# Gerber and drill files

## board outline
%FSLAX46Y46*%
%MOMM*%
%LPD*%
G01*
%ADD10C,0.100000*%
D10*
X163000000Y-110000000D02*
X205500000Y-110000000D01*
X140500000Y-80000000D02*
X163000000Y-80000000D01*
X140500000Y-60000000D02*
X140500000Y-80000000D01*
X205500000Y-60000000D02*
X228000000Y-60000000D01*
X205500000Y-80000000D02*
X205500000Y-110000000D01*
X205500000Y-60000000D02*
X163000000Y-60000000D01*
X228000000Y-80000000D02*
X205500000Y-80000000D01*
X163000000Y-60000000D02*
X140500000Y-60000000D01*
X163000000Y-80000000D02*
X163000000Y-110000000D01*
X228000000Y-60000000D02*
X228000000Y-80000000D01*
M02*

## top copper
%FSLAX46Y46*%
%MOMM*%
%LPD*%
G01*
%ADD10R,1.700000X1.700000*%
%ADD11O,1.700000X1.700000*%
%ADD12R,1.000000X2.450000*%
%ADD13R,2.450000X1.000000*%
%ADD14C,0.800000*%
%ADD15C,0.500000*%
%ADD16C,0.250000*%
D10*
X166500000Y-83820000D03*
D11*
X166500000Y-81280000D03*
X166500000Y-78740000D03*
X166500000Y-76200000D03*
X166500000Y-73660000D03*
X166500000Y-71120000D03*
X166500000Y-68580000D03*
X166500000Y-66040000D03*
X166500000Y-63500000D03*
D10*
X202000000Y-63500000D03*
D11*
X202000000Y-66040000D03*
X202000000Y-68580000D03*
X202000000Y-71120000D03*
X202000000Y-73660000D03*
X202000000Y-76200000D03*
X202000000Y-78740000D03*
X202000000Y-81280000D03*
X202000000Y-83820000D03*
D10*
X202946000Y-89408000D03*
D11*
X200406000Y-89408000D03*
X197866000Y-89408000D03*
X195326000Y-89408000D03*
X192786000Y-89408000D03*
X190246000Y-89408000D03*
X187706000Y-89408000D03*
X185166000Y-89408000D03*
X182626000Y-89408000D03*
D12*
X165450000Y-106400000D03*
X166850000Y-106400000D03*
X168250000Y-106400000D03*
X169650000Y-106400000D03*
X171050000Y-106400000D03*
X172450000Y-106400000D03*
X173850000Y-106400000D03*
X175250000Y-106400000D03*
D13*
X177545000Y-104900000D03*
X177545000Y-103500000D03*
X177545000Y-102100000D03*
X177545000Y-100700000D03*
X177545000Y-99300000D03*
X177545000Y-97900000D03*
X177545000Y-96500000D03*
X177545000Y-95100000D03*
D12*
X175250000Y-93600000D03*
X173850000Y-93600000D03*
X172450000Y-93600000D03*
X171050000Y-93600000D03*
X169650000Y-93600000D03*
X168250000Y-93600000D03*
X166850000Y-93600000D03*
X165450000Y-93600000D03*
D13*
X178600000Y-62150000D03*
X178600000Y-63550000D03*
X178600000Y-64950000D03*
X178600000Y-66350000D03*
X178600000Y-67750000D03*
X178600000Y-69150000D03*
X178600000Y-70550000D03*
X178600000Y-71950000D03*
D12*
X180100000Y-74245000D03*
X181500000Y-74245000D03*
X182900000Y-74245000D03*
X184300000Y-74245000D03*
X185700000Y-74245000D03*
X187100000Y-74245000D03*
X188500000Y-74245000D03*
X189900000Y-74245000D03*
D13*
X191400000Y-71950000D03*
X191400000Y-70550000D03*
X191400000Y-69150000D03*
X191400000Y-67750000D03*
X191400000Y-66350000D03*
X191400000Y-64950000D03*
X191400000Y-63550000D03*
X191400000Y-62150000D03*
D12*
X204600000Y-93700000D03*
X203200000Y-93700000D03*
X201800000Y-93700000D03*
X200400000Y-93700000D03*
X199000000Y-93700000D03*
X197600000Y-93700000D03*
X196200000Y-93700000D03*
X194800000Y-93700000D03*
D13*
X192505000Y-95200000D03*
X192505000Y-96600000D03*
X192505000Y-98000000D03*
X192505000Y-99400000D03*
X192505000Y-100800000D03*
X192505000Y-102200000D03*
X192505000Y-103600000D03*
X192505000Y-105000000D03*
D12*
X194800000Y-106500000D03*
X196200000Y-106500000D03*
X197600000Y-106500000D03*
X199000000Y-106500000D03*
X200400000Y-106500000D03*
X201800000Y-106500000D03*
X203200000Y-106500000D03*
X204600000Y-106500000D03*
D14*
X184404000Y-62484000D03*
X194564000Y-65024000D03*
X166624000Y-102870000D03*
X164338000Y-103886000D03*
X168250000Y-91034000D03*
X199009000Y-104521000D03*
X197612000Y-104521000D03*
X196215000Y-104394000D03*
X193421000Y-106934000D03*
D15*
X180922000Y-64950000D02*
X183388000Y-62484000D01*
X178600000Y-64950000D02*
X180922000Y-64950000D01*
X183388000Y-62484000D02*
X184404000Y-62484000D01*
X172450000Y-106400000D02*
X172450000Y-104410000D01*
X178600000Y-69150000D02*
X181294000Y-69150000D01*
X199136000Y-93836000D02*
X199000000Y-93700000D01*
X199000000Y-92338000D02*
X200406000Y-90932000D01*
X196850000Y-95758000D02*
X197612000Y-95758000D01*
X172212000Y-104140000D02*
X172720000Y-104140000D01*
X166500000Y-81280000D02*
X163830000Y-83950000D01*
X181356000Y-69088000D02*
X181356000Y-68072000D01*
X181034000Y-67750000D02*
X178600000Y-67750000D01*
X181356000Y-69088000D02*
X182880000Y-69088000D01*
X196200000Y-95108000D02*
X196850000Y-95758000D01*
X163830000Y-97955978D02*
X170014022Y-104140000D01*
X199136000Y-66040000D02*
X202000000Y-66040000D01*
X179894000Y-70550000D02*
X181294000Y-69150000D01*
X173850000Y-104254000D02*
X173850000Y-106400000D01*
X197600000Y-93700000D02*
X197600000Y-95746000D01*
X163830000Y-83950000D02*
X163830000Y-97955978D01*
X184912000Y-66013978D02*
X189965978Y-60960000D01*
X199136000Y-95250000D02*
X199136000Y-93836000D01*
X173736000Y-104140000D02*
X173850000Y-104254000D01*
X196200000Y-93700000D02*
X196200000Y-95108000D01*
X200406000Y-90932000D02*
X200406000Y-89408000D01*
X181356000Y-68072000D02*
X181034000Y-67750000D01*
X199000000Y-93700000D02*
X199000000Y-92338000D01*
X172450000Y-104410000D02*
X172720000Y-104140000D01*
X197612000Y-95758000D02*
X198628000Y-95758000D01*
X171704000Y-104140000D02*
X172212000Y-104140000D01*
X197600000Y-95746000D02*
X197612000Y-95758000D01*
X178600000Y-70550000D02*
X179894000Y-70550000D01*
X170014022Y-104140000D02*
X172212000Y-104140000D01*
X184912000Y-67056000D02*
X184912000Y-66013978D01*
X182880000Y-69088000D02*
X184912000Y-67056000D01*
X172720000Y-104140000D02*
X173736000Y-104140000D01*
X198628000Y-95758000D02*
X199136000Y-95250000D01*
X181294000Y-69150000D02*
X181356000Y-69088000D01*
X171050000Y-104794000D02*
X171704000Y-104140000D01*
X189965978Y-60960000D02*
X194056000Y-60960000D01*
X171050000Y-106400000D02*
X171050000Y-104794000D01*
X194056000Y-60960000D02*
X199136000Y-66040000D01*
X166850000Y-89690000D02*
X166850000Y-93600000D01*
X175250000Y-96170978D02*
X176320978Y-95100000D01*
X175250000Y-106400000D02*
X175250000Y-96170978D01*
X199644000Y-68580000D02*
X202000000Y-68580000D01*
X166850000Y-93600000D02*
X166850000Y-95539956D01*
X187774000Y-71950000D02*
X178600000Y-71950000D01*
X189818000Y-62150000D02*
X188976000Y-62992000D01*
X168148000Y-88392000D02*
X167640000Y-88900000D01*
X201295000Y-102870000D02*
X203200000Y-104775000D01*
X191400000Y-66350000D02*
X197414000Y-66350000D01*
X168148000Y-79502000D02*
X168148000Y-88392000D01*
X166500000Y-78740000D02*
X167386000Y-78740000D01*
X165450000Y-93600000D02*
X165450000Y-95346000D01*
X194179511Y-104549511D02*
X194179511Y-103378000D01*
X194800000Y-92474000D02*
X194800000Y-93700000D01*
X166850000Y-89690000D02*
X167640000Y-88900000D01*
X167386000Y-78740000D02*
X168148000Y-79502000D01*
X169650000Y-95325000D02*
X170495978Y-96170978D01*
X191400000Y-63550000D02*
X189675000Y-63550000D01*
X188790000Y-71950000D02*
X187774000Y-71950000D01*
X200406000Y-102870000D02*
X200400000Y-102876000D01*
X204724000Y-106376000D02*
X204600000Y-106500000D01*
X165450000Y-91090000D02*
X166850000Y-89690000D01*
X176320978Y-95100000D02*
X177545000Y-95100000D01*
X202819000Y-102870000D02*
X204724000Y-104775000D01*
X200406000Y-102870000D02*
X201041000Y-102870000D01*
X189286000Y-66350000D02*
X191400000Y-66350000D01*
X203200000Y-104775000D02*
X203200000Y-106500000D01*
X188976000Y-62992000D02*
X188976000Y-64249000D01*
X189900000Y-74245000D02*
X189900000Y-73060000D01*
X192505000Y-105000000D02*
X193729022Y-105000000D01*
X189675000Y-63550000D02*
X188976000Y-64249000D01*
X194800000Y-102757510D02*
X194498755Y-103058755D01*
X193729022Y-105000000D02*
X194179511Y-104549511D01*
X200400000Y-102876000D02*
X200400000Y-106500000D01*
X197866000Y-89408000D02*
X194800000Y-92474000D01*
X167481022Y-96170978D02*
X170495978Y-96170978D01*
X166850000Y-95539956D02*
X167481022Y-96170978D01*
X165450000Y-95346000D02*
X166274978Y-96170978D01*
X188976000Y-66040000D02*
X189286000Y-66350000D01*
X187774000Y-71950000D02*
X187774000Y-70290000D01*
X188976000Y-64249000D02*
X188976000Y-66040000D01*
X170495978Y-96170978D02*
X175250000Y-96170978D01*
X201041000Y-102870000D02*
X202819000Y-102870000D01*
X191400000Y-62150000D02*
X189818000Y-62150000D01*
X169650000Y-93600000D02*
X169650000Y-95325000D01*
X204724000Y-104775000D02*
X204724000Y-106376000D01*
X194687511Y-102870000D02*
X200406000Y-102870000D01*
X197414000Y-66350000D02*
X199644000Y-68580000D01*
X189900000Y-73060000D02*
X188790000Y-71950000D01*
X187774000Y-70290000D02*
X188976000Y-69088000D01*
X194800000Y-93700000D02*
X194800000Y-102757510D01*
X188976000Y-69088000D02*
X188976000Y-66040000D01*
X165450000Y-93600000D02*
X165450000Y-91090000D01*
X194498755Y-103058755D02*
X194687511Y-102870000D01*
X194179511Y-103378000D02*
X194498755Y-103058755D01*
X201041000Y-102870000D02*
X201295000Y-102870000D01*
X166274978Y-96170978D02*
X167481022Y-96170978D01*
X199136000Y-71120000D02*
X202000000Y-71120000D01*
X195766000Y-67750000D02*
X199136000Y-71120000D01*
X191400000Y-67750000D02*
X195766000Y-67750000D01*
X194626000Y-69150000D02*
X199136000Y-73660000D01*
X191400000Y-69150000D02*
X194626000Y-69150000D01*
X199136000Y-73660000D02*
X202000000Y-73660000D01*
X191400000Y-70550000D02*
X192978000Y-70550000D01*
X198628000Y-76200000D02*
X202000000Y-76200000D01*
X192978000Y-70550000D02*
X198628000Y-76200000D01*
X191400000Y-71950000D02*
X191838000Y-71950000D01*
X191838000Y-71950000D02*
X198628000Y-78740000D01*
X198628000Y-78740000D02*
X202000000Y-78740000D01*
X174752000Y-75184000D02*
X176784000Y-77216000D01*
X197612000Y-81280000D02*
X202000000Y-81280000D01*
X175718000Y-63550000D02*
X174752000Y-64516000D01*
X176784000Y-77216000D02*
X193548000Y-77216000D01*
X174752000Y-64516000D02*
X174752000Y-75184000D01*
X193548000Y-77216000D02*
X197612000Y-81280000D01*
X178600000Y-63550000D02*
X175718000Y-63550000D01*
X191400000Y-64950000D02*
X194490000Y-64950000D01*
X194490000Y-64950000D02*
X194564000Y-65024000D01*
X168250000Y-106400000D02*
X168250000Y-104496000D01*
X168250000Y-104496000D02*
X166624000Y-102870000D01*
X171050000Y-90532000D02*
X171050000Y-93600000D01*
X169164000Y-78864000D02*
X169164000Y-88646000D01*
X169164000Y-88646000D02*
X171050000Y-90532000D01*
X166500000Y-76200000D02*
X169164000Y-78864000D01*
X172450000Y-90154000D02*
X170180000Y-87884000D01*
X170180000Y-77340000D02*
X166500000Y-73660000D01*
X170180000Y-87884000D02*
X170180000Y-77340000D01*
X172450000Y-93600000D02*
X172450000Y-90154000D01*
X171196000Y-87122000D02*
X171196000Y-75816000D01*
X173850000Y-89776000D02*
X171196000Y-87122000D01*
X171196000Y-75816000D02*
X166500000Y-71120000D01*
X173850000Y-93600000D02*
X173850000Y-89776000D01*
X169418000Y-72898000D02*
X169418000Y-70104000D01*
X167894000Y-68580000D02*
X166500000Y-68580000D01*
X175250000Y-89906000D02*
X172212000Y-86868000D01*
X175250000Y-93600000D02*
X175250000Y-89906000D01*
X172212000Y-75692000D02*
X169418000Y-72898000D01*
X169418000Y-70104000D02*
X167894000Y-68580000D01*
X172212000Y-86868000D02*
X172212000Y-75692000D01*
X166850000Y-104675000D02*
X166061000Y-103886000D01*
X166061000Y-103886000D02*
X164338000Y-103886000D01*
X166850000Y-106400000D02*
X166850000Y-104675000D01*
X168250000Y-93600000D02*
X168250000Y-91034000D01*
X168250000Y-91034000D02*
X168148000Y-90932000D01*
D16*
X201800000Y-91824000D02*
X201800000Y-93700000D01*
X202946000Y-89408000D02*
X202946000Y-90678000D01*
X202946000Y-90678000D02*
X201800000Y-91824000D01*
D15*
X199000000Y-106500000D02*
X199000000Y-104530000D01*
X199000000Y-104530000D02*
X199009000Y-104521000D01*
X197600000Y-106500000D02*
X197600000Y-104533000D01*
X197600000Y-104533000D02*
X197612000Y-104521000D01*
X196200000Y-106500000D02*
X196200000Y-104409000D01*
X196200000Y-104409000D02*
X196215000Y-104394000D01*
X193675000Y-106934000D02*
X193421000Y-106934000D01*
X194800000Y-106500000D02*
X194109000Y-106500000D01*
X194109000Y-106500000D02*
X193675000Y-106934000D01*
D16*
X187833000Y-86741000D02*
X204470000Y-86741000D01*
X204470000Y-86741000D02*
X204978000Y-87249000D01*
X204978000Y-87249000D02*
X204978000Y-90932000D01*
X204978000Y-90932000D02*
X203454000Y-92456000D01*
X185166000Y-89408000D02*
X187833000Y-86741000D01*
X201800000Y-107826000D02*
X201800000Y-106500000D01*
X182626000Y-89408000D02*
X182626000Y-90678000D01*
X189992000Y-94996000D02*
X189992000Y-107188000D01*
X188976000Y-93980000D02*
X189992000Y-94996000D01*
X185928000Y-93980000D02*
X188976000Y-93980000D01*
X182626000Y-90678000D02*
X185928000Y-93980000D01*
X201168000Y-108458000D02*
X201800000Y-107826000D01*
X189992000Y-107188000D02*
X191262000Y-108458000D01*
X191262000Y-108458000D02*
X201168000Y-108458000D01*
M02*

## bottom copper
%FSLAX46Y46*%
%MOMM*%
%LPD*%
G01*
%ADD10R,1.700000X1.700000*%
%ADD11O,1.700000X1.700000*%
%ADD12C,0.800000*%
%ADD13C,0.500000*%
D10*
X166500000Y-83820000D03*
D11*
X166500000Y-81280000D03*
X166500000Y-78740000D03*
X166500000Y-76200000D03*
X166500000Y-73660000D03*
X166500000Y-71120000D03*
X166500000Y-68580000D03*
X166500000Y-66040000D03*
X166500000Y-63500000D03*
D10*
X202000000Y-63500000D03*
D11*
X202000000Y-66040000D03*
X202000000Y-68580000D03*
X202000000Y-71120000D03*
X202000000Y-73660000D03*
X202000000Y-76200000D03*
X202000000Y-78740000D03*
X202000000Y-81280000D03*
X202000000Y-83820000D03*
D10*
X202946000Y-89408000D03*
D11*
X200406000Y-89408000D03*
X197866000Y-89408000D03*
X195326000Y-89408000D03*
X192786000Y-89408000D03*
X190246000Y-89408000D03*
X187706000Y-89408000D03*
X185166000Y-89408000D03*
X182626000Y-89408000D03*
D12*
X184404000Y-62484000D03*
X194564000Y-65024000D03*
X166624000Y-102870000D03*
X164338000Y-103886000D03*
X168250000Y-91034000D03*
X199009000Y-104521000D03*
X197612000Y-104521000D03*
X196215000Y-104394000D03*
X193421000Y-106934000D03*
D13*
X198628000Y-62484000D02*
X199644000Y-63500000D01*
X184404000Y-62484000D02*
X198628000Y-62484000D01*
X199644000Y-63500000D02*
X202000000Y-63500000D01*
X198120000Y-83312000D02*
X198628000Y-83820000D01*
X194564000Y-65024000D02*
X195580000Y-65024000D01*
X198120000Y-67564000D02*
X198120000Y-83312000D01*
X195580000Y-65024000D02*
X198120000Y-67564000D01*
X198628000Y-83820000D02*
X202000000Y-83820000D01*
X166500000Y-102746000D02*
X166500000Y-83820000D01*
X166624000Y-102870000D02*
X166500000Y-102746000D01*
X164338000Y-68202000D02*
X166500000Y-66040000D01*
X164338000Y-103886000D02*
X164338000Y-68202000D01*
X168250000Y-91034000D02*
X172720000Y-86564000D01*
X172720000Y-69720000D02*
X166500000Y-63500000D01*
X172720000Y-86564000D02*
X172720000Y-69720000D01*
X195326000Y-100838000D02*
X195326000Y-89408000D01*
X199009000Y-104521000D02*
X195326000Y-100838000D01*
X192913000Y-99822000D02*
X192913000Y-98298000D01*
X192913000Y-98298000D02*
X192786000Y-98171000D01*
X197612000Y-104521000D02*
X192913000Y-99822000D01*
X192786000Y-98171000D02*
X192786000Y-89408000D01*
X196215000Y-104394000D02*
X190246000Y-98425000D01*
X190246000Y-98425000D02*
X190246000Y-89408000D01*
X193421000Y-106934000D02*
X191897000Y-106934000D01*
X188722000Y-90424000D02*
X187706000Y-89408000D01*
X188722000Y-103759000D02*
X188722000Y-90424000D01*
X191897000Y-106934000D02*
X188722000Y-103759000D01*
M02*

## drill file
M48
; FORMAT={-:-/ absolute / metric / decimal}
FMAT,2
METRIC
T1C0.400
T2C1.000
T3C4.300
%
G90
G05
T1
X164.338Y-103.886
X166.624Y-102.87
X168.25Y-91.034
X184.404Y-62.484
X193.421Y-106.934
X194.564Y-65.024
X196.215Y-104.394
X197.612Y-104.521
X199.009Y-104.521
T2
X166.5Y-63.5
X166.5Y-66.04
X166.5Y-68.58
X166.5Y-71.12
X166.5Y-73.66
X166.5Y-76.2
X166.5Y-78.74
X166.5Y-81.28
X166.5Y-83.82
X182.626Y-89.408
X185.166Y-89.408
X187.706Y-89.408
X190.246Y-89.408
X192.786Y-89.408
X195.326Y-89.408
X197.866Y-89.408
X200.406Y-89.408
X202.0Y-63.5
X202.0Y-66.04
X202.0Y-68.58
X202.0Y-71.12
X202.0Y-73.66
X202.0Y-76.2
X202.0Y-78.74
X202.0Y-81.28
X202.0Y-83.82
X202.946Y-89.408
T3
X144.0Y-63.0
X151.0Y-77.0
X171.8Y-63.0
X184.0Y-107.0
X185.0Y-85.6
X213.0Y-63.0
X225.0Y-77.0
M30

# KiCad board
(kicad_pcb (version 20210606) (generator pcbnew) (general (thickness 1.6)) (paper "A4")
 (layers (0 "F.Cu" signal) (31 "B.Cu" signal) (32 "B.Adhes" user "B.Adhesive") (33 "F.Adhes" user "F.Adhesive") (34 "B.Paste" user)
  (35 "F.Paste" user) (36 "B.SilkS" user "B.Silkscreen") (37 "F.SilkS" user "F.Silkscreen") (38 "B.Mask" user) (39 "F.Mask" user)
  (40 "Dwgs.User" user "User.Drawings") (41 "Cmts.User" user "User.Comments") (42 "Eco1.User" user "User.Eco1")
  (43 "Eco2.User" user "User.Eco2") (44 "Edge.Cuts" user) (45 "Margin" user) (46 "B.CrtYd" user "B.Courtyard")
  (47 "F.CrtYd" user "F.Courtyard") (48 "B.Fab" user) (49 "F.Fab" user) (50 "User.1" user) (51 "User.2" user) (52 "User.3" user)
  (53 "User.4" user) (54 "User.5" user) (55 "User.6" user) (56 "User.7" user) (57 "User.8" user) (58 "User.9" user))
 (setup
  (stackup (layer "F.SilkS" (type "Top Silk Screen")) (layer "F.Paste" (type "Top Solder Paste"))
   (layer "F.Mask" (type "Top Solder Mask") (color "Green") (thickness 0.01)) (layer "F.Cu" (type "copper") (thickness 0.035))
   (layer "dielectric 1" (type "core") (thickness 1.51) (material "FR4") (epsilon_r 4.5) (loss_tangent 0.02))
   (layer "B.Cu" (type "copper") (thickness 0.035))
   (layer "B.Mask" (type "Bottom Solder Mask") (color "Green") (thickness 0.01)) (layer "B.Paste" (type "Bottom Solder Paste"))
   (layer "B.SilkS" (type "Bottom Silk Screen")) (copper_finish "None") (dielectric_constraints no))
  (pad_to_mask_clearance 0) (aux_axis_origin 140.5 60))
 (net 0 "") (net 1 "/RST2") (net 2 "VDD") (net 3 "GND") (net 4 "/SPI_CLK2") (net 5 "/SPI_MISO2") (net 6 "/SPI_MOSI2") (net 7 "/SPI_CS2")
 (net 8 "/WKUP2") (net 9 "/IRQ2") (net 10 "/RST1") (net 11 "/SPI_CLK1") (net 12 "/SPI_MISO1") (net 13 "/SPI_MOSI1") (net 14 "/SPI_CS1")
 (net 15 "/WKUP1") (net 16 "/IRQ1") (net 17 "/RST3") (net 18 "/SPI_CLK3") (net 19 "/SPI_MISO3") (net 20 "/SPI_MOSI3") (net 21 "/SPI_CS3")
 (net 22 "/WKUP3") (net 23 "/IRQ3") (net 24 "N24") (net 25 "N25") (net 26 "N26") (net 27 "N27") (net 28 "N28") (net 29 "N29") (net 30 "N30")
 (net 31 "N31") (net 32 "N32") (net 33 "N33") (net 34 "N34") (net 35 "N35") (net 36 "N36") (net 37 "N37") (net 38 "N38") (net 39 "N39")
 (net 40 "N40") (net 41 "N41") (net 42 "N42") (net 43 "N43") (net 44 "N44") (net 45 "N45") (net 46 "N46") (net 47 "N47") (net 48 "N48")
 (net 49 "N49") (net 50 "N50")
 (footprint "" (layer "F.Cu") (at 151 77)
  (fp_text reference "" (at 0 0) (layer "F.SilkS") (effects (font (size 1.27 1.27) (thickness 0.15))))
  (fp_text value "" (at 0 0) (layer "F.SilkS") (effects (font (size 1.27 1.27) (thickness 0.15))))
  (pad "1" np_thru_hole circle locked (at 0 0) (size 4.3 4.3) (drill 4.3) (layers *.Cu *.Mask)))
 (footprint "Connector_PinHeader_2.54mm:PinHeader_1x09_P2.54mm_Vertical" (layer "F.Cu") (at 166.5 83.82 180)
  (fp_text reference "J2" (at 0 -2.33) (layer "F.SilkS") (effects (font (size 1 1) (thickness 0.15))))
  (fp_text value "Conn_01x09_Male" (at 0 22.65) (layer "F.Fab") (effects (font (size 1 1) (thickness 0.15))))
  (pad "1" thru_hole rect locked (at 0 0 180) (size 1.7 1.7) (drill 1) (layers *.Cu *.Mask) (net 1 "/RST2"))
  (pad "2" thru_hole oval locked (at 0 2.54 180) (size 1.7 1.7) (drill 1) (layers *.Cu *.Mask) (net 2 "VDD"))
  (pad "3" thru_hole oval locked (at 0 5.08 180) (size 1.7 1.7) (drill 1) (layers *.Cu *.Mask) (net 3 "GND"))
  (pad "4" thru_hole oval locked (at 0 7.62 180) (size 1.7 1.7) (drill 1) (layers *.Cu *.Mask) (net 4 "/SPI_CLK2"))
  (pad "5" thru_hole oval locked (at 0 10.16 180) (size 1.7 1.7) (drill 1) (layers *.Cu *.Mask) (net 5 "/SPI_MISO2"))
  (pad "6" thru_hole oval locked (at 0 12.7 180) (size 1.7 1.7) (drill 1) (layers *.Cu *.Mask) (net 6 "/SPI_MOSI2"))
  (pad "7" thru_hole oval locked (at 0 15.24 180) (size 1.7 1.7) (drill 1) (layers *.Cu *.Mask) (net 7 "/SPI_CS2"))
  (pad "8" thru_hole oval locked (at 0 17.78 180) (size 1.7 1.7) (drill 1) (layers *.Cu *.Mask) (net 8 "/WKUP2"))
  (pad "9" thru_hole oval locked (at 0 20.32 180) (size 1.7 1.7) (drill 1) (layers *.Cu *.Mask) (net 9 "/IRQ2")))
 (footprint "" (layer "F.Cu") (at 213 63)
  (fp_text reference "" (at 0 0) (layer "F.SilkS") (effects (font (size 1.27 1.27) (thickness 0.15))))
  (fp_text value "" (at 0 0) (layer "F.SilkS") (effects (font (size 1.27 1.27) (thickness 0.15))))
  (pad "1" np_thru_hole circle locked (at 0 0) (size 4.3 4.3) (drill 4.3) (layers *.Cu *.Mask)))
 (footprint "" (layer "F.Cu") (at 185 85.6)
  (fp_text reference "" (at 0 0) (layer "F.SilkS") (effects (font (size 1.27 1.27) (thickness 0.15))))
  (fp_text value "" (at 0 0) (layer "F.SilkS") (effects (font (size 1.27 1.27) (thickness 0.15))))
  (pad "1" np_thru_hole circle locked (at 0 0) (size 4.3 4.3) (drill 4.3) (layers *.Cu *.Mask)))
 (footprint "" (layer "F.Cu") (at 225 77)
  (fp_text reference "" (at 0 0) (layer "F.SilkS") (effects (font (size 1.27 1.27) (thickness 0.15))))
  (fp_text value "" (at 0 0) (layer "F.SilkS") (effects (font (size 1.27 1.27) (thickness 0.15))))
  (pad "1" np_thru_hole circle locked (at 0 0) (size 4.3 4.3) (drill 4.3) (layers *.Cu *.Mask)))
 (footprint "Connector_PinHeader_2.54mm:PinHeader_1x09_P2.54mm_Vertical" (layer "F.Cu") (at 202 63.5)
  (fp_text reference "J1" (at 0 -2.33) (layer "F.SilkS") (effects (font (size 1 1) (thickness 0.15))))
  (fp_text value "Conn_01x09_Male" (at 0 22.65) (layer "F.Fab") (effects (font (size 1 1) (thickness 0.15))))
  (pad "1" thru_hole rect locked (at 0 0) (size 1.7 1.7) (drill 1) (layers *.Cu *.Mask) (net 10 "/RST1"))
  (pad "2" thru_hole oval locked (at 0 2.54) (size 1.7 1.7) (drill 1) (layers *.Cu *.Mask) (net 2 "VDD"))
  (pad "3" thru_hole oval locked (at 0 5.08) (size 1.7 1.7) (drill 1) (layers *.Cu *.Mask) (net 3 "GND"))
  (pad "4" thru_hole oval locked (at 0 7.62) (size 1.7 1.7) (drill 1) (layers *.Cu *.Mask) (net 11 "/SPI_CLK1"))
  (pad "5" thru_hole oval locked (at 0 10.16) (size 1.7 1.7) (drill 1) (layers *.Cu *.Mask) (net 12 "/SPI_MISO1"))
  (pad "6" thru_hole oval locked (at 0 12.7) (size 1.7 1.7) (drill 1) (layers *.Cu *.Mask) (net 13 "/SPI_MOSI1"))
  (pad "7" thru_hole oval locked (at 0 15.24) (size 1.7 1.7) (drill 1) (layers *.Cu *.Mask) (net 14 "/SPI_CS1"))
  (pad "8" thru_hole oval locked (at 0 17.78) (size 1.7 1.7) (drill 1) (layers *.Cu *.Mask) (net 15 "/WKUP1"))
  (pad "9" thru_hole oval locked (at 0 20.32) (size 1.7 1.7) (drill 1) (layers *.Cu *.Mask) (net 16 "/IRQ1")))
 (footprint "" (layer "F.Cu") (at 184 107)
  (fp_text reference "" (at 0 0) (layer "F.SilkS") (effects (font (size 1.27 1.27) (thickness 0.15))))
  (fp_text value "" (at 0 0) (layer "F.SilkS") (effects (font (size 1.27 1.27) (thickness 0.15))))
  (pad "1" np_thru_hole circle locked (at 0 0) (size 4.3 4.3) (drill 4.3) (layers *.Cu *.Mask)))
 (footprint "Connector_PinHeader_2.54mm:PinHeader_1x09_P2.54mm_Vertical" (layer "F.Cu") (at 202.946 89.408 -90)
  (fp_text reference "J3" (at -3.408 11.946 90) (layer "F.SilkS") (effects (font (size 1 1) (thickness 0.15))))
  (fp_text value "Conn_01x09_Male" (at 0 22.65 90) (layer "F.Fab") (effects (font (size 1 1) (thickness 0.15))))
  (pad "1" thru_hole rect locked (at 0 0 270) (size 1.7 1.7) (drill 1) (layers *.Cu *.Mask) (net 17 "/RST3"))
  (pad "2" thru_hole oval locked (at 0 2.54 270) (size 1.7 1.7) (drill 1) (layers *.Cu *.Mask) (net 2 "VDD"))
  (pad "3" thru_hole oval locked (at 0 5.08 270) (size 1.7 1.7) (drill 1) (layers *.Cu *.Mask) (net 3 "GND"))
  (pad "4" thru_hole oval locked (at 0 7.62 270) (size 1.7 1.7) (drill 1) (layers *.Cu *.Mask) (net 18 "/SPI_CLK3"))
  (pad "5" thru_hole oval locked (at 0 10.16 270) (size 1.7 1.7) (drill 1) (layers *.Cu *.Mask) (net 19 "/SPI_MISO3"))
  (pad "6" thru_hole oval locked (at 0 12.7 270) (size 1.7 1.7) (drill 1) (layers *.Cu *.Mask) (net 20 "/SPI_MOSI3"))
  (pad "7" thru_hole oval locked (at 0 15.24 270) (size 1.7 1.7) (drill 1) (layers *.Cu *.Mask) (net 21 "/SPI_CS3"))
  (pad "8" thru_hole oval locked (at 0 17.78 270) (size 1.7 1.7) (drill 1) (layers *.Cu *.Mask) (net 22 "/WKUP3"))
  (pad "9" thru_hole oval locked (at 0 20.32 270) (size 1.7 1.7) (drill 1) (layers *.Cu *.Mask) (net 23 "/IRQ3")))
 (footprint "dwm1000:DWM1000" (layer "F.Cu") (at 167.25 100 90)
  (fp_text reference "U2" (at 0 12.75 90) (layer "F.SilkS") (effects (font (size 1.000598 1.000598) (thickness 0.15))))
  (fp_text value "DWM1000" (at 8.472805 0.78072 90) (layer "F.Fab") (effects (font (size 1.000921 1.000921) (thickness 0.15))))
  (pad "1" smd rect locked (at -6.4 -1.8 90) (size 2.45 1) (layers "F.Cu" "F.Paste" "F.Mask") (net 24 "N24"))
  (pad "2" smd rect locked (at -6.4 -0.4 90) (size 2.45 1) (layers "F.Cu" "F.Paste" "F.Mask") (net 8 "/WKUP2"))
  (pad "3" smd rect locked (at -6.4 1 90) (size 2.45 1) (layers "F.Cu" "F.Paste" "F.Mask") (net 1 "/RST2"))
  (pad "4" smd rect locked (at -6.4 2.4 90) (size 2.45 1) (layers "F.Cu" "F.Paste" "F.Mask") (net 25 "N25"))
  (pad "5" smd rect locked (at -6.4 3.8 90) (size 2.45 1) (layers "F.Cu" "F.Paste" "F.Mask") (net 2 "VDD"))
  (pad "6" smd rect locked (at -6.4 5.2 90) (size 2.45 1) (layers "F.Cu" "F.Paste" "F.Mask") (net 2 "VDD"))
  (pad "7" smd rect locked (at -6.4 6.6 90) (size 2.45 1) (layers "F.Cu" "F.Paste" "F.Mask") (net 2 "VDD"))
  (pad "8" smd rect locked (at -6.4 8 90) (size 2.45 1) (layers "F.Cu" "F.Paste" "F.Mask") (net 3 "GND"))
  (pad "9" smd rect locked (at -4.9 10.295 90) (size 1 2.45) (layers "F.Cu" "F.Paste" "F.Mask") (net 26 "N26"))
  (pad "10" smd rect locked (at -3.5 10.295 90) (size 1 2.45) (layers "F.Cu" "F.Paste" "F.Mask") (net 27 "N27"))
  (pad "11" smd rect locked (at -2.1 10.295 90) (size 1 2.45) (layers "F.Cu" "F.Paste" "F.Mask") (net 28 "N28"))
  (pad "12" smd rect locked (at -0.7 10.295 90) (size 1 2.45) (layers "F.Cu" "F.Paste" "F.Mask") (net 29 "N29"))
  (pad "13" smd rect locked (at 0.7 10.295 90) (size 1 2.45) (layers "F.Cu" "F.Paste" "F.Mask") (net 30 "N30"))
  (pad "14" smd rect locked (at 2.1 10.295 90) (size 1 2.45) (layers "F.Cu" "F.Paste" "F.Mask") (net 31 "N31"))
  (pad "15" smd rect locked (at 3.5 10.295 90) (size 1 2.45) (layers "F.Cu" "F.Paste" "F.Mask") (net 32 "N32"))
  (pad "16" smd rect locked (at 4.9 10.295 90) (size 1 2.45) (layers "F.Cu" "F.Paste" "F.Mask") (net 3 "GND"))
  (pad "17" smd rect locked (at 6.4 8 90) (size 2.45 1) (layers "F.Cu" "F.Paste" "F.Mask") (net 7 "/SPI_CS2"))
  (pad "18" smd rect locked (at 6.4 6.6 90) (size 2.45 1) (layers "F.Cu" "F.Paste" "F.Mask") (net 6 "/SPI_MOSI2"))
  (pad "19" smd rect locked (at 6.4 5.2 90) (size 2.45 1) (layers "F.Cu" "F.Paste" "F.Mask") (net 5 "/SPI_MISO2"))
  (pad "20" smd rect locked (at 6.4 3.8 90) (size 2.45 1) (layers "F.Cu" "F.Paste" "F.Mask") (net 4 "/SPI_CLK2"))
  (pad "21" smd rect locked (at 6.4 2.4 90) (size 2.45 1) (layers "F.Cu" "F.Paste" "F.Mask") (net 3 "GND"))
  (pad "22" smd rect locked (at 6.4 1 90) (size 2.45 1) (layers "F.Cu" "F.Paste" "F.Mask") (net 9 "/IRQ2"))
  (pad "23" smd rect locked (at 6.4 -0.4 90) (size 2.45 1) (layers "F.Cu" "F.Paste" "F.Mask") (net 3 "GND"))
  (pad "24" smd rect locked (at 6.4 -1.8 90) (size 2.45 1) (layers "F.Cu" "F.Paste" "F.Mask") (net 3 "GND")))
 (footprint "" (layer "F.Cu") (at 144 63)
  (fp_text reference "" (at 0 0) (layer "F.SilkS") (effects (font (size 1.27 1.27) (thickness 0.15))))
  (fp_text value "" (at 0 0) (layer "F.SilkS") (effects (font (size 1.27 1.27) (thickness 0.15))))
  (pad "1" np_thru_hole circle locked (at 0 0) (size 4.3 4.3) (drill 4.3) (layers *.Cu *.Mask)))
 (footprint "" (layer "F.Cu") (at 171.8 63)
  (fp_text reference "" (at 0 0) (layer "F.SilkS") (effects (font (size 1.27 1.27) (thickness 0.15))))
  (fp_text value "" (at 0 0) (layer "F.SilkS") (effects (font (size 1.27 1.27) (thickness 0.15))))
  (pad "1" np_thru_hole circle locked (at 0 0) (size 4.3 4.3) (drill 4.3) (layers *.Cu *.Mask)))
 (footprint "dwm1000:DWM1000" (layer "F.Cu") (at 185 63.95)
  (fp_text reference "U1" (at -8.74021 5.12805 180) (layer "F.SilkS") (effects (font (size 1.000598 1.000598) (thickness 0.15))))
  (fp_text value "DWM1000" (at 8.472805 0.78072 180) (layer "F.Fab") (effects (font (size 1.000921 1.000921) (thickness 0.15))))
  (pad "1" smd rect locked (at -6.4 -1.8) (size 2.45 1) (layers "F.Cu" "F.Paste" "F.Mask") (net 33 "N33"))
  (pad "2" smd rect locked (at -6.4 -0.4) (size 2.45 1) (layers "F.Cu" "F.Paste" "F.Mask") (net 15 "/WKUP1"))
  (pad "3" smd rect locked (at -6.4 1) (size 2.45 1) (layers "F.Cu" "F.Paste" "F.Mask") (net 10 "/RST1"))
  (pad "4" smd rect locked (at -6.4 2.4) (size 2.45 1) (layers "F.Cu" "F.Paste" "F.Mask") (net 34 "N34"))
  (pad "5" smd rect locked (at -6.4 3.8) (size 2.45 1) (layers "F.Cu" "F.Paste" "F.Mask") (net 2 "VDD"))
  (pad "6" smd rect locked (at -6.4 5.2) (size 2.45 1) (layers "F.Cu" "F.Paste" "F.Mask") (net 2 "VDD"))
  (pad "7" smd rect locked (at -6.4 6.6) (size 2.45 1) (layers "F.Cu" "F.Paste" "F.Mask") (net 2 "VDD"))
  (pad "8" smd rect locked (at -6.4 8) (size 2.45 1) (layers "F.Cu" "F.Paste" "F.Mask") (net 3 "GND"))
  (pad "9" smd rect locked (at -4.9 10.295) (size 1 2.45) (layers "F.Cu" "F.Paste" "F.Mask") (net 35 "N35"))
  (pad "10" smd rect locked (at -3.5 10.295) (size 1 2.45) (layers "F.Cu" "F.Paste" "F.Mask") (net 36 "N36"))
  (pad "11" smd rect locked (at -2.1 10.295) (size 1 2.45) (layers "F.Cu" "F.Paste" "F.Mask") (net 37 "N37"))
  (pad "12" smd rect locked (at -0.7 10.295) (size 1 2.45) (layers "F.Cu" "F.Paste" "F.Mask") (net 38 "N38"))
  (pad "13" smd rect locked (at 0.7 10.295) (size 1 2.45) (layers "F.Cu" "F.Paste" "F.Mask") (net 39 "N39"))
  (pad "14" smd rect locked (at 2.1 10.295) (size 1 2.45) (layers "F.Cu" "F.Paste" "F.Mask") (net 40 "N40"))
  (pad "15" smd rect locked (at 3.5 10.295) (size 1 2.45) (layers "F.Cu" "F.Paste" "F.Mask") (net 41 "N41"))
  (pad "16" smd rect locked (at 4.9 10.295) (size 1 2.45) (layers "F.Cu" "F.Paste" "F.Mask") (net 3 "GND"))
  (pad "17" smd rect locked (at 6.4 8) (size 2.45 1) (layers "F.Cu" "F.Paste" "F.Mask") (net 14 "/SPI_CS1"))
  (pad "18" smd rect locked (at 6.4 6.6) (size 2.45 1) (layers "F.Cu" "F.Paste" "F.Mask") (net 13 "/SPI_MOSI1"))
  (pad "19" smd rect locked (at 6.4 5.2) (size 2.45 1) (layers "F.Cu" "F.Paste" "F.Mask") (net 12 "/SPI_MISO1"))
  (pad "20" smd rect locked (at 6.4 3.8) (size 2.45 1) (layers "F.Cu" "F.Paste" "F.Mask") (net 11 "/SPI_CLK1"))
  (pad "21" smd rect locked (at 6.4 2.4) (size 2.45 1) (layers "F.Cu" "F.Paste" "F.Mask") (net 3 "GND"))
  (pad "22" smd rect locked (at 6.4 1) (size 2.45 1) (layers "F.Cu" "F.Paste" "F.Mask") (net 16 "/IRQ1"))
  (pad "23" smd rect locked (at 6.4 -0.4) (size 2.45 1) (layers "F.Cu" "F.Paste" "F.Mask") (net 3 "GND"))
  (pad "24" smd rect locked (at 6.4 -1.8) (size 2.45 1) (layers "F.Cu" "F.Paste" "F.Mask") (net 3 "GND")))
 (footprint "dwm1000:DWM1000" (layer "F.Cu") (at 202.8 100.1 -90)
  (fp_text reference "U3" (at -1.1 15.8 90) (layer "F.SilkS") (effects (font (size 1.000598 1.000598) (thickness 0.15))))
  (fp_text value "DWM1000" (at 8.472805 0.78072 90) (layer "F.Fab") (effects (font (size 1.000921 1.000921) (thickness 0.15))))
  (pad "1" smd rect locked (at -6.4 -1.8 270) (size 2.45 1) (layers "F.Cu" "F.Paste" "F.Mask") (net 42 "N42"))
  (pad "2" smd rect locked (at -6.4 -0.4 270) (size 2.45 1) (layers "F.Cu" "F.Paste" "F.Mask") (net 22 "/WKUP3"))
  (pad "3" smd rect locked (at -6.4 1 270) (size 2.45 1) (layers "F.Cu" "F.Paste" "F.Mask") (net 17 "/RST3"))
  (pad "4" smd rect locked (at -6.4 2.4 270) (size 2.45 1) (layers "F.Cu" "F.Paste" "F.Mask") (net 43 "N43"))
  (pad "5" smd rect locked (at -6.4 3.8 270) (size 2.45 1) (layers "F.Cu" "F.Paste" "F.Mask") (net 2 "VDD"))
  (pad "6" smd rect locked (at -6.4 5.2 270) (size 2.45 1) (layers "F.Cu" "F.Paste" "F.Mask") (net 2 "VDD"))
  (pad "7" smd rect locked (at -6.4 6.6 270) (size 2.45 1) (layers "F.Cu" "F.Paste" "F.Mask") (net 2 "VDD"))
  (pad "8" smd rect locked (at -6.4 8 270) (size 2.45 1) (layers "F.Cu" "F.Paste" "F.Mask") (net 3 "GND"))
  (pad "9" smd rect locked (at -4.9 10.295 270) (size 1 2.45) (layers "F.Cu" "F.Paste" "F.Mask") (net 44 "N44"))
  (pad "10" smd rect locked (at -3.5 10.295 270) (size 1 2.45) (layers "F.Cu" "F.Paste" "F.Mask") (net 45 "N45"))
  (pad "11" smd rect locked (at -2.1 10.295 270) (size 1 2.45) (layers "F.Cu" "F.Paste" "F.Mask") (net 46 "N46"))
  (pad "12" smd rect locked (at -0.7 10.295 270) (size 1 2.45) (layers "F.Cu" "F.Paste" "F.Mask") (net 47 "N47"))
  (pad "13" smd rect locked (at 0.7 10.295 270) (size 1 2.45) (layers "F.Cu" "F.Paste" "F.Mask") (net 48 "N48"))
  (pad "14" smd rect locked (at 2.1 10.295 270) (size 1 2.45) (layers "F.Cu" "F.Paste" "F.Mask") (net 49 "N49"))
  (pad "15" smd rect locked (at 3.5 10.295 270) (size 1 2.45) (layers "F.Cu" "F.Paste" "F.Mask") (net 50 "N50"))
  (pad "16" smd rect locked (at 4.9 10.295 270) (size 1 2.45) (layers "F.Cu" "F.Paste" "F.Mask") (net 3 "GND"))
  (pad "17" smd rect locked (at 6.4 8 270) (size 2.45 1) (layers "F.Cu" "F.Paste" "F.Mask") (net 21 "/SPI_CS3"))
  (pad "18" smd rect locked (at 6.4 6.6 270) (size 2.45 1) (layers "F.Cu" "F.Paste" "F.Mask") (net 20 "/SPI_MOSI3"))
  (pad "19" smd rect locked (at 6.4 5.2 270) (size 2.45 1) (layers "F.Cu" "F.Paste" "F.Mask") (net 19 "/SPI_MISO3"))
  (pad "20" smd rect locked (at 6.4 3.8 270) (size 2.45 1) (layers "F.Cu" "F.Paste" "F.Mask") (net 18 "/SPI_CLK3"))
  (pad "21" smd rect locked (at 6.4 2.4 270) (size 2.45 1) (layers "F.Cu" "F.Paste" "F.Mask") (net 3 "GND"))
  (pad "22" smd rect locked (at 6.4 1 270) (size 2.45 1) (layers "F.Cu" "F.Paste" "F.Mask") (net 23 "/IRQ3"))
  (pad "23" smd rect locked (at 6.4 -0.4 270) (size 2.45 1) (layers "F.Cu" "F.Paste" "F.Mask") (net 3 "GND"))
  (pad "24" smd rect locked (at 6.4 -1.8 270) (size 2.45 1) (layers "F.Cu" "F.Paste" "F.Mask") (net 3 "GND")))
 (gr_line (start 163 110) (end 205.5 110) (layer "Edge.Cuts") (width 0.1))
 (gr_line (start 140.5 80) (end 163 80) (layer "Edge.Cuts") (width 0.1))
 (gr_line (start 140.5 60) (end 140.5 80) (layer "Edge.Cuts") (width 0.1))
 (gr_line (start 205.5 60) (end 228 60) (layer "Edge.Cuts") (width 0.1))
 (gr_line (start 205.5 80) (end 205.5 110) (layer "Edge.Cuts") (width 0.1))
 (gr_line (start 205.5 60) (end 163 60) (layer "Edge.Cuts") (width 0.1))
 (gr_line (start 228 80) (end 205.5 80) (layer "Edge.Cuts") (width 0.1))
 (gr_line (start 163 60) (end 140.5 60) (layer "Edge.Cuts") (width 0.1))
 (gr_line (start 163 80) (end 163 110) (layer "Edge.Cuts") (width 0.1))
 (gr_line (start 228 60) (end 228 80) (layer "Edge.Cuts") (width 0.1))
 (segment (start 180.922 64.95) (end 183.388 62.484) (width 0.5) (layer "F.Cu") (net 10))
 (segment (start 178.6 64.95) (end 180.922 64.95) (width 0.5) (layer "F.Cu") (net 10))
 (segment (start 183.388 62.484) (end 184.404 62.484) (width 0.5) (layer "F.Cu") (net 10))
 (via (at 184.404 62.484) (size 0.8) (drill 0.4) (layers "F.Cu" "B.Cu") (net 10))
 (segment (start 198.628 62.484) (end 199.644 63.5) (width 0.5) (layer "B.Cu") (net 10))
 (segment (start 184.404 62.484) (end 198.628 62.484) (width 0.5) (layer "B.Cu") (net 10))
 (segment (start 199.644 63.5) (end 202 63.5) (width 0.5) (layer "B.Cu") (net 10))
 (segment (start 172.45 106.4) (end 172.45 104.41) (width 0.5) (layer "F.Cu") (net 2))
 (segment (start 178.6 69.15) (end 181.294 69.15) (width 0.5) (layer "F.Cu") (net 2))
 (segment (start 199.136 93.836) (end 199 93.7) (width 0.5) (layer "F.Cu") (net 2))
 (segment (start 199 92.338) (end 200.406 90.932) (width 0.5) (layer "F.Cu") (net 2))
 (segment (start 196.85 95.758) (end 197.612 95.758) (width 0.5) (layer "F.Cu") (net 2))
 (segment (start 172.212 104.14) (end 172.72 104.14) (width 0.5) (layer "F.Cu") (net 2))
 (segment (start 166.5 81.28) (end 163.83 83.95) (width 0.5) (layer "F.Cu") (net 2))
 (segment (start 181.356 69.088) (end 181.356 68.072) (width 0.5) (layer "F.Cu") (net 2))
 (segment (start 181.034 67.75) (end 178.6 67.75) (width 0.5) (layer "F.Cu") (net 2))
 (segment (start 181.356 69.088) (end 182.88 69.088) (width 0.5) (layer "F.Cu") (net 2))
 (segment (start 196.2 95.108) (end 196.85 95.758) (width 0.5) (layer "F.Cu") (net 2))
 (segment (start 163.83 97.955978) (end 170.014022 104.14) (width 0.5) (layer "F.Cu") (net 2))
 (segment (start 199.136 66.04) (end 202 66.04) (width 0.5) (layer "F.Cu") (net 2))
 (segment (start 179.894 70.55) (end 181.294 69.15) (width 0.5) (layer "F.Cu") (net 2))
 (segment (start 173.85 104.254) (end 173.85 106.4) (width 0.5) (layer "F.Cu") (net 2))
 (segment (start 197.6 93.7) (end 197.6 95.746) (width 0.5) (layer "F.Cu") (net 2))
 (segment (start 163.83 83.95) (end 163.83 97.955978) (width 0.5) (layer "F.Cu") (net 2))
 (segment (start 184.912 66.013978) (end 189.965978 60.96) (width 0.5) (layer "F.Cu") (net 2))
 (segment (start 199.136 95.25) (end 199.136 93.836) (width 0.5) (layer "F.Cu") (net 2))
 (segment (start 173.736 104.14) (end 173.85 104.254) (width 0.5) (layer "F.Cu") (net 2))
 (segment (start 196.2 93.7) (end 196.2 95.108) (width 0.5) (layer "F.Cu") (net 2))
 (segment (start 200.406 90.932) (end 200.406 89.408) (width 0.5) (layer "F.Cu") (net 2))
 (segment (start 181.356 68.072) (end 181.034 67.75) (width 0.5) (layer "F.Cu") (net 2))
 (segment (start 199 93.7) (end 199 92.338) (width 0.5) (layer "F.Cu") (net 2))
 (segment (start 172.45 104.41) (end 172.72 104.14) (width 0.5) (layer "F.Cu") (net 2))
 (segment (start 197.612 95.758) (end 198.628 95.758) (width 0.5) (layer "F.Cu") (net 2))
 (segment (start 171.704 104.14) (end 172.212 104.14) (width 0.5) (layer "F.Cu") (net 2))
 (segment (start 197.6 95.746) (end 197.612 95.758) (width 0.5) (layer "F.Cu") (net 2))
 (segment (start 178.6 70.55) (end 179.894 70.55) (width 0.5) (layer "F.Cu") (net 2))
 (segment (start 170.014022 104.14) (end 172.212 104.14) (width 0.5) (layer "F.Cu") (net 2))
 (segment (start 184.912 67.056) (end 184.912 66.013978) (width 0.5) (layer "F.Cu") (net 2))
 (segment (start 182.88 69.088) (end 184.912 67.056) (width 0.5) (layer "F.Cu") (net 2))
 (segment (start 172.72 104.14) (end 173.736 104.14) (width 0.5) (layer "F.Cu") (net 2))
 (segment (start 198.628 95.758) (end 199.136 95.25) (width 0.5) (layer "F.Cu") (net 2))
 (segment (start 181.294 69.15) (end 181.356 69.088) (width 0.5) (layer "F.Cu") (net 2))
 (segment (start 171.05 104.794) (end 171.704 104.14) (width 0.5) (layer "F.Cu") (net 2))
 (segment (start 189.965978 60.96) (end 194.056 60.96) (width 0.5) (layer "F.Cu") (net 2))
 (segment (start 171.05 106.4) (end 171.05 104.794) (width 0.5) (layer "F.Cu") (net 2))
 (segment (start 194.056 60.96) (end 199.136 66.04) (width 0.5) (layer "F.Cu") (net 2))
 (segment (start 166.85 89.69) (end 166.85 93.6) (width 0.5) (layer "F.Cu") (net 3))
 (segment (start 175.25 96.170978) (end 176.320978 95.1) (width 0.5) (layer "F.Cu") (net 3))
 (segment (start 175.25 106.4) (end 175.25 96.170978) (width 0.5) (layer "F.Cu") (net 3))
 (segment (start 199.644 68.58) (end 202 68.58) (width 0.5) (layer "F.Cu") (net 3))
 (segment (start 166.85 93.6) (end 166.85 95.539956) (width 0.5) (layer "F.Cu") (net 3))
 (segment (start 187.774 71.95) (end 178.6 71.95) (width 0.5) (layer "F.Cu") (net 3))
 (segment (start 189.818 62.15) (end 188.976 62.992) (width 0.5) (layer "F.Cu") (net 3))
 (segment (start 168.148 88.392) (end 167.64 88.9) (width 0.5) (layer "F.Cu") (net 3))
 (segment (start 201.295 102.87) (end 203.2 104.775) (width 0.5) (layer "F.Cu") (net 3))
 (segment (start 191.4 66.35) (end 197.414 66.35) (width 0.5) (layer "F.Cu") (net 3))
 (segment (start 168.148 79.502) (end 168.148 88.392) (width 0.5) (layer "F.Cu") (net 3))
 (segment (start 166.5 78.74) (end 167.386 78.74) (width 0.5) (layer "F.Cu") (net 3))
 (segment (start 165.45 93.6) (end 165.45 95.346) (width 0.5) (layer "F.Cu") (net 3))
 (segment (start 194.179511 104.549511) (end 194.179511 103.378) (width 0.5) (layer "F.Cu") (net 3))
 (segment (start 194.8 92.474) (end 194.8 93.7) (width 0.5) (layer "F.Cu") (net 3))
 (segment (start 166.85 89.69) (end 167.64 88.9) (width 0.5) (layer "F.Cu") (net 3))
 (segment (start 167.386 78.74) (end 168.148 79.502) (width 0.5) (layer "F.Cu") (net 3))
 (segment (start 169.65 95.325) (end 170.495978 96.170978) (width 0.5) (layer "F.Cu") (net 3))
 (segment (start 191.4 63.55) (end 189.675 63.55) (width 0.5) (layer "F.Cu") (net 3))
 (segment (start 188.79 71.95) (end 187.774 71.95) (width 0.5) (layer "F.Cu") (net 3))
 (segment (start 200.406 102.87) (end 200.4 102.876) (width 0.5) (layer "F.Cu") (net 3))
 (segment (start 204.724 106.376) (end 204.6 106.5) (width 0.5) (layer "F.Cu") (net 3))
 (segment (start 165.45 91.09) (end 166.85 89.69) (width 0.5) (layer "F.Cu") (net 3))
 (segment (start 176.320978 95.1) (end 177.545 95.1) (width 0.5) (layer "F.Cu") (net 3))
 (segment (start 202.819 102.87) (end 204.724 104.775) (width 0.5) (layer "F.Cu") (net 3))
 (segment (start 200.406 102.87) (end 201.041 102.87) (width 0.5) (layer "F.Cu") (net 3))
 (segment (start 189.286 66.35) (end 191.4 66.35) (width 0.5) (layer "F.Cu") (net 3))
 (segment (start 203.2 104.775) (end 203.2 106.5) (width 0.5) (layer "F.Cu") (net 3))
 (segment (start 188.976 62.992) (end 188.976 64.249) (width 0.5) (layer "F.Cu") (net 3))
 (segment (start 189.9 74.245) (end 189.9 73.06) (width 0.5) (layer "F.Cu") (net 3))
 (segment (start 192.505 105) (end 193.729022 105) (width 0.5) (layer "F.Cu") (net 3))
 (segment (start 189.675 63.55) (end 188.976 64.249) (width 0.5) (layer "F.Cu") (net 3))
 (segment (start 194.8 102.75751) (end 194.498755 103.058755) (width 0.5) (layer "F.Cu") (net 3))
 (segment (start 193.729022 105) (end 194.179511 104.549511) (width 0.5) (layer "F.Cu") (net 3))
 (segment (start 200.4 102.876) (end 200.4 106.5) (width 0.5) (layer "F.Cu") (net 3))
 (segment (start 197.866 89.408) (end 194.8 92.474) (width 0.5) (layer "F.Cu") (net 3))
 (segment (start 167.481022 96.170978) (end 170.495978 96.170978) (width 0.5) (layer "F.Cu") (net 3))
 (segment (start 166.85 95.539956) (end 167.481022 96.170978) (width 0.5) (layer "F.Cu") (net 3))
 (segment (start 165.45 95.346) (end 166.274978 96.170978) (width 0.5) (layer "F.Cu") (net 3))
 (segment (start 188.976 66.04) (end 189.286 66.35) (width 0.5) (layer "F.Cu") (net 3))
 (segment (start 187.774 71.95) (end 187.774 70.29) (width 0.5) (layer "F.Cu") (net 3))
 (segment (start 188.976 64.249) (end 188.976 66.04) (width 0.5) (layer "F.Cu") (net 3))
 (segment (start 170.495978 96.170978) (end 175.25 96.170978) (width 0.5) (layer "F.Cu") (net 3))
 (segment (start 201.041 102.87) (end 202.819 102.87) (width 0.5) (layer "F.Cu") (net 3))
 (segment (start 191.4 62.15) (end 189.818 62.15) (width 0.5) (layer "F.Cu") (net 3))
 (segment (start 169.65 93.6) (end 169.65 95.325) (width 0.5) (layer "F.Cu") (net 3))
 (segment (start 204.724 104.775) (end 204.724 106.376) (width 0.5) (layer "F.Cu") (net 3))
 (segment (start 194.687511 102.87) (end 200.406 102.87) (width 0.5) (layer "F.Cu") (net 3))
 (segment (start 197.414 66.35) (end 199.644 68.58) (width 0.5) (layer "F.Cu") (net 3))
 (segment (start 189.9 73.06) (end 188.79 71.95) (width 0.5) (layer "F.Cu") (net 3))
 (segment (start 187.774 70.29) (end 188.976 69.088) (width 0.5) (layer "F.Cu") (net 3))
 (segment (start 194.8 93.7) (end 194.8 102.75751) (width 0.5) (layer "F.Cu") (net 3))
 (segment (start 188.976 69.088) (end 188.976 66.04) (width 0.5) (layer "F.Cu") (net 3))
 (segment (start 165.45 93.6) (end 165.45 91.09) (width 0.5) (layer "F.Cu") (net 3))
 (segment (start 194.498755 103.058755) (end 194.687511 102.87) (width 0.5) (layer "F.Cu") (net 3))
 (segment (start 194.179511 103.378) (end 194.498755 103.058755) (width 0.5) (layer "F.Cu") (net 3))
 (segment (start 201.041 102.87) (end 201.295 102.87) (width 0.5) (layer "F.Cu") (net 3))
 (segment (start 166.274978 96.170978) (end 167.481022 96.170978) (width 0.5) (layer "F.Cu") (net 3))
 (segment (start 199.136 71.12) (end 202 71.12) (width 0.5) (layer "F.Cu") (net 11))
 (segment (start 195.766 67.75) (end 199.136 71.12) (width 0.5) (layer "F.Cu") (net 11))
 (segment (start 191.4 67.75) (end 195.766 67.75) (width 0.5) (layer "F.Cu") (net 11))
 (segment (start 194.626 69.15) (end 199.136 73.66) (width 0.5) (layer "F.Cu") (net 12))
 (segment (start 191.4 69.15) (end 194.626 69.15) (width 0.5) (layer "F.Cu") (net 12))
 (segment (start 199.136 73.66) (end 202 73.66) (width 0.5) (layer "F.Cu") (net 12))
 (segment (start 191.4 70.55) (end 192.978 70.55) (width 0.5) (layer "F.Cu") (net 13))
 (segment (start 198.628 76.2) (end 202 76.2) (width 0.5) (layer "F.Cu") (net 13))
 (segment (start 192.978 70.55) (end 198.628 76.2) (width 0.5) (layer "F.Cu") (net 13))
 (segment (start 191.4 71.95) (end 191.838 71.95) (width 0.5) (layer "F.Cu") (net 14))
 (segment (start 191.838 71.95) (end 198.628 78.74) (width 0.5) (layer "F.Cu") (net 14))
 (segment (start 198.628 78.74) (end 202 78.74) (width 0.5) (layer "F.Cu") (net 14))
 (segment (start 174.752 75.184) (end 176.784 77.216) (width 0.5) (layer "F.Cu") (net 15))
 (segment (start 197.612 81.28) (end 202 81.28) (width 0.5) (layer "F.Cu") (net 15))
 (segment (start 175.718 63.55) (end 174.752 64.516) (width 0.5) (layer "F.Cu") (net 15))
 (segment (start 176.784 77.216) (end 193.548 77.216) (width 0.5) (layer "F.Cu") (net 15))
 (segment (start 174.752 64.516) (end 174.752 75.184) (width 0.5) (layer "F.Cu") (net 15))
 (segment (start 193.548 77.216) (end 197.612 81.28) (width 0.5) (layer "F.Cu") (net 15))
 (segment (start 178.6 63.55) (end 175.718 63.55) (width 0.5) (layer "F.Cu") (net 15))
 (segment (start 191.4 64.95) (end 194.49 64.95) (width 0.5) (layer "F.Cu") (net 16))
 (segment (start 194.49 64.95) (end 194.564 65.024) (width 0.5) (layer "F.Cu") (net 16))
 (via (at 194.564 65.024) (size 0.8) (drill 0.4) (layers "F.Cu" "B.Cu") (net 16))
 (segment (start 198.12 83.312) (end 198.628 83.82) (width 0.5) (layer "B.Cu") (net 16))
 (segment (start 194.564 65.024) (end 195.58 65.024) (width 0.5) (layer "B.Cu") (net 16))
 (segment (start 198.12 67.564) (end 198.12 83.312) (width 0.5) (layer "B.Cu") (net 16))
 (segment (start 195.58 65.024) (end 198.12 67.564) (width 0.5) (layer "B.Cu") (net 16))
 (segment (start 198.628 83.82) (end 202 83.82) (width 0.5) (layer "B.Cu") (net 16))
 (segment (start 168.25 106.4) (end 168.25 104.496) (width 0.5) (layer "F.Cu") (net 1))
 (segment (start 168.25 104.496) (end 166.624 102.87) (width 0.5) (layer "F.Cu") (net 1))
 (via (at 166.624 102.87) (size 0.8) (drill 0.4) (layers "F.Cu" "B.Cu") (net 1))
 (segment (start 166.5 102.746) (end 166.5 83.82) (width 0.5) (layer "B.Cu") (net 1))
 (segment (start 166.624 102.87) (end 166.5 102.746) (width 0.5) (layer "B.Cu") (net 1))
 (segment (start 171.05 90.532) (end 171.05 93.6) (width 0.5) (layer "F.Cu") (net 4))
 (segment (start 169.164 78.864) (end 169.164 88.646) (width 0.5) (layer "F.Cu") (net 4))
 (segment (start 169.164 88.646) (end 171.05 90.532) (width 0.5) (layer "F.Cu") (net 4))
 (segment (start 166.5 76.2) (end 169.164 78.864) (width 0.5) (layer "F.Cu") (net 4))
 (segment (start 172.45 90.154) (end 170.18 87.884) (width 0.5) (layer "F.Cu") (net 5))
 (segment (start 170.18 77.34) (end 166.5 73.66) (width 0.5) (layer "F.Cu") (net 5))
 (segment (start 170.18 87.884) (end 170.18 77.34) (width 0.5) (layer "F.Cu") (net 5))
 (segment (start 172.45 93.6) (end 172.45 90.154) (width 0.5) (layer "F.Cu") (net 5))
 (segment (start 171.196 87.122) (end 171.196 75.816) (width 0.5) (layer "F.Cu") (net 6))
 (segment (start 173.85 89.776) (end 171.196 87.122) (width 0.5) (layer "F.Cu") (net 6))
 (segment (start 171.196 75.816) (end 166.5 71.12) (width 0.5) (layer "F.Cu") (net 6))
 (segment (start 173.85 93.6) (end 173.85 89.776) (width 0.5) (layer "F.Cu") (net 6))
 (segment (start 169.418 72.898) (end 169.418 70.104) (width 0.5) (layer "F.Cu") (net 7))
 (segment (start 167.894 68.58) (end 166.5 68.58) (width 0.5) (layer "F.Cu") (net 7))
 (segment (start 175.25 89.906) (end 172.212 86.868) (width 0.5) (layer "F.Cu") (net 7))
 (segment (start 175.25 93.6) (end 175.25 89.906) (width 0.5) (layer "F.Cu") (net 7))
 (segment (start 172.212 75.692) (end 169.418 72.898) (width 0.5) (layer "F.Cu") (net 7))
 (segment (start 169.418 70.104) (end 167.894 68.58) (width 0.5) (layer "F.Cu") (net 7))
 (segment (start 172.212 86.868) (end 172.212 75.692) (width 0.5) (layer "F.Cu") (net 7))
 (segment (start 166.85 104.675) (end 166.061 103.886) (width 0.5) (layer "F.Cu") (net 8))
 (segment (start 166.061 103.886) (end 164.338 103.886) (width 0.5) (layer "F.Cu") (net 8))
 (segment (start 166.85 106.4) (end 166.85 104.675) (width 0.5) (layer "F.Cu") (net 8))
 (via (at 164.338 103.886) (size 0.8) (drill 0.4) (layers "F.Cu" "B.Cu") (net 8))
 (segment (start 164.338 68.202) (end 166.5 66.04) (width 0.5) (layer "B.Cu") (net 8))
 (segment (start 164.338 103.886) (end 164.338 68.202) (width 0.5) (layer "B.Cu") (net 8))
 (segment (start 168.25 93.6) (end 168.25 91.034) (width 0.5) (layer "F.Cu") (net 9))
 (segment (start 168.25 91.034) (end 168.148 90.932) (width 0.5) (layer "F.Cu") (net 9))
 (via (at 168.25 91.034) (size 0.8) (drill 0.4) (layers "F.Cu" "B.Cu") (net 9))
 (segment (start 168.25 91.034) (end 172.72 86.564) (width 0.5) (layer "B.Cu") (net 9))
 (segment (start 172.72 69.72) (end 166.5 63.5) (width 0.5) (layer "B.Cu") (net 9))
 (segment (start 172.72 86.564) (end 172.72 69.72) (width 0.5) (layer "B.Cu") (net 9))
 (segment (start 201.8 91.824) (end 201.8 93.7) (width 0.25) (layer "F.Cu") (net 17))
 (segment (start 202.946 89.408) (end 202.946 90.678) (width 0.25) (layer "F.Cu") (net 17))
 (segment (start 202.946 90.678) (end 201.8 91.824) (width 0.25) (layer "F.Cu") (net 17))
 (segment (start 199 106.5) (end 199 104.53) (width 0.5) (layer "F.Cu") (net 18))
 (segment (start 199 104.53) (end 199.009 104.521) (width 0.5) (layer "F.Cu") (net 18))
 (via (at 199.009 104.521) (size 0.8) (drill 0.4) (layers "F.Cu" "B.Cu") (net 18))
 (segment (start 195.326 100.838) (end 195.326 89.408) (width 0.5) (layer "B.Cu") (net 18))
 (segment (start 199.009 104.521) (end 195.326 100.838) (width 0.5) (layer "B.Cu") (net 18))
 (segment (start 197.6 106.5) (end 197.6 104.533) (width 0.5) (layer "F.Cu") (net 19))
 (segment (start 197.6 104.533) (end 197.612 104.521) (width 0.5) (layer "F.Cu") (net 19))
 (via (at 197.612 104.521) (size 0.8) (drill 0.4) (layers "F.Cu" "B.Cu") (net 19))
 (segment (start 192.913 99.822) (end 192.913 98.298) (width 0.5) (layer "B.Cu") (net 19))
 (segment (start 192.913 98.298) (end 192.786 98.171) (width 0.5) (layer "B.Cu") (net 19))
 (segment (start 197.612 104.521) (end 192.913 99.822) (width 0.5) (layer "B.Cu") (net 19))
 (segment (start 192.786 98.171) (end 192.786 89.408) (width 0.5) (layer "B.Cu") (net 19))
 (segment (start 196.2 106.5) (end 196.2 104.409) (width 0.5) (layer "F.Cu") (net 20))
 (segment (start 196.2 104.409) (end 196.215 104.394) (width 0.5) (layer "F.Cu") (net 20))
 (via (at 196.215 104.394) (size 0.8) (drill 0.4) (layers "F.Cu" "B.Cu") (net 20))
 (segment (start 196.215 104.394) (end 190.246 98.425) (width 0.5) (layer "B.Cu") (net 20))
 (segment (start 190.246 98.425) (end 190.246 89.408) (width 0.5) (layer "B.Cu") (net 20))
 (segment (start 193.675 106.934) (end 193.421 106.934) (width 0.5) (layer "F.Cu") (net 21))
 (segment (start 194.8 106.5) (end 194.109 106.5) (width 0.5) (layer "F.Cu") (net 21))
 (segment (start 194.109 106.5) (end 193.675 106.934) (width 0.5) (layer "F.Cu") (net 21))
 (via (at 193.421 106.934) (size 0.8) (drill 0.4) (layers "F.Cu" "B.Cu") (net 21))
 (segment (start 193.421 106.934) (end 191.897 106.934) (width 0.5) (layer "B.Cu") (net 21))
 (segment (start 188.722 90.424) (end 187.706 89.408) (width 0.5) (layer "B.Cu") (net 21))
 (segment (start 188.722 103.759) (end 188.722 90.424) (width 0.5) (layer "B.Cu") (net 21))
 (segment (start 191.897 106.934) (end 188.722 103.759) (width 0.5) (layer "B.Cu") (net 21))
 (segment (start 187.833 86.741) (end 204.47 86.741) (width 0.25) (layer "F.Cu") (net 22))
 (segment (start 204.47 86.741) (end 204.978 87.249) (width 0.25) (layer "F.Cu") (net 22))
 (segment (start 204.978 87.249) (end 204.978 90.932) (width 0.25) (layer "F.Cu") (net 22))
 (segment (start 204.978 90.932) (end 203.454 92.456) (width 0.25) (layer "F.Cu") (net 22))
 (segment (start 185.166 89.408) (end 187.833 86.741) (width 0.25) (layer "F.Cu") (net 22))
 (segment (start 201.8 107.826) (end 201.8 106.5) (width 0.25) (layer "F.Cu") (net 23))
 (segment (start 182.626 89.408) (end 182.626 90.678) (width 0.25) (layer "F.Cu") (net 23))
 (segment (start 189.992 94.996) (end 189.992 107.188) (width 0.25) (layer "F.Cu") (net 23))
 (segment (start 188.976 93.98) (end 189.992 94.996) (width 0.25) (layer "F.Cu") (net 23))
 (segment (start 185.928 93.98) (end 188.976 93.98) (width 0.25) (layer "F.Cu") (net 23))
 (segment (start 182.626 90.678) (end 185.928 93.98) (width 0.25) (layer "F.Cu") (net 23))
 (segment (start 201.168 108.458) (end 201.8 107.826) (width 0.25) (layer "F.Cu") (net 23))
 (segment (start 189.992 107.188) (end 191.262 108.458) (width 0.25) (layer "F.Cu") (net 23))
 (segment (start 191.262 108.458) (end 201.168 108.458) (width 0.25) (layer "F.Cu") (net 23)))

